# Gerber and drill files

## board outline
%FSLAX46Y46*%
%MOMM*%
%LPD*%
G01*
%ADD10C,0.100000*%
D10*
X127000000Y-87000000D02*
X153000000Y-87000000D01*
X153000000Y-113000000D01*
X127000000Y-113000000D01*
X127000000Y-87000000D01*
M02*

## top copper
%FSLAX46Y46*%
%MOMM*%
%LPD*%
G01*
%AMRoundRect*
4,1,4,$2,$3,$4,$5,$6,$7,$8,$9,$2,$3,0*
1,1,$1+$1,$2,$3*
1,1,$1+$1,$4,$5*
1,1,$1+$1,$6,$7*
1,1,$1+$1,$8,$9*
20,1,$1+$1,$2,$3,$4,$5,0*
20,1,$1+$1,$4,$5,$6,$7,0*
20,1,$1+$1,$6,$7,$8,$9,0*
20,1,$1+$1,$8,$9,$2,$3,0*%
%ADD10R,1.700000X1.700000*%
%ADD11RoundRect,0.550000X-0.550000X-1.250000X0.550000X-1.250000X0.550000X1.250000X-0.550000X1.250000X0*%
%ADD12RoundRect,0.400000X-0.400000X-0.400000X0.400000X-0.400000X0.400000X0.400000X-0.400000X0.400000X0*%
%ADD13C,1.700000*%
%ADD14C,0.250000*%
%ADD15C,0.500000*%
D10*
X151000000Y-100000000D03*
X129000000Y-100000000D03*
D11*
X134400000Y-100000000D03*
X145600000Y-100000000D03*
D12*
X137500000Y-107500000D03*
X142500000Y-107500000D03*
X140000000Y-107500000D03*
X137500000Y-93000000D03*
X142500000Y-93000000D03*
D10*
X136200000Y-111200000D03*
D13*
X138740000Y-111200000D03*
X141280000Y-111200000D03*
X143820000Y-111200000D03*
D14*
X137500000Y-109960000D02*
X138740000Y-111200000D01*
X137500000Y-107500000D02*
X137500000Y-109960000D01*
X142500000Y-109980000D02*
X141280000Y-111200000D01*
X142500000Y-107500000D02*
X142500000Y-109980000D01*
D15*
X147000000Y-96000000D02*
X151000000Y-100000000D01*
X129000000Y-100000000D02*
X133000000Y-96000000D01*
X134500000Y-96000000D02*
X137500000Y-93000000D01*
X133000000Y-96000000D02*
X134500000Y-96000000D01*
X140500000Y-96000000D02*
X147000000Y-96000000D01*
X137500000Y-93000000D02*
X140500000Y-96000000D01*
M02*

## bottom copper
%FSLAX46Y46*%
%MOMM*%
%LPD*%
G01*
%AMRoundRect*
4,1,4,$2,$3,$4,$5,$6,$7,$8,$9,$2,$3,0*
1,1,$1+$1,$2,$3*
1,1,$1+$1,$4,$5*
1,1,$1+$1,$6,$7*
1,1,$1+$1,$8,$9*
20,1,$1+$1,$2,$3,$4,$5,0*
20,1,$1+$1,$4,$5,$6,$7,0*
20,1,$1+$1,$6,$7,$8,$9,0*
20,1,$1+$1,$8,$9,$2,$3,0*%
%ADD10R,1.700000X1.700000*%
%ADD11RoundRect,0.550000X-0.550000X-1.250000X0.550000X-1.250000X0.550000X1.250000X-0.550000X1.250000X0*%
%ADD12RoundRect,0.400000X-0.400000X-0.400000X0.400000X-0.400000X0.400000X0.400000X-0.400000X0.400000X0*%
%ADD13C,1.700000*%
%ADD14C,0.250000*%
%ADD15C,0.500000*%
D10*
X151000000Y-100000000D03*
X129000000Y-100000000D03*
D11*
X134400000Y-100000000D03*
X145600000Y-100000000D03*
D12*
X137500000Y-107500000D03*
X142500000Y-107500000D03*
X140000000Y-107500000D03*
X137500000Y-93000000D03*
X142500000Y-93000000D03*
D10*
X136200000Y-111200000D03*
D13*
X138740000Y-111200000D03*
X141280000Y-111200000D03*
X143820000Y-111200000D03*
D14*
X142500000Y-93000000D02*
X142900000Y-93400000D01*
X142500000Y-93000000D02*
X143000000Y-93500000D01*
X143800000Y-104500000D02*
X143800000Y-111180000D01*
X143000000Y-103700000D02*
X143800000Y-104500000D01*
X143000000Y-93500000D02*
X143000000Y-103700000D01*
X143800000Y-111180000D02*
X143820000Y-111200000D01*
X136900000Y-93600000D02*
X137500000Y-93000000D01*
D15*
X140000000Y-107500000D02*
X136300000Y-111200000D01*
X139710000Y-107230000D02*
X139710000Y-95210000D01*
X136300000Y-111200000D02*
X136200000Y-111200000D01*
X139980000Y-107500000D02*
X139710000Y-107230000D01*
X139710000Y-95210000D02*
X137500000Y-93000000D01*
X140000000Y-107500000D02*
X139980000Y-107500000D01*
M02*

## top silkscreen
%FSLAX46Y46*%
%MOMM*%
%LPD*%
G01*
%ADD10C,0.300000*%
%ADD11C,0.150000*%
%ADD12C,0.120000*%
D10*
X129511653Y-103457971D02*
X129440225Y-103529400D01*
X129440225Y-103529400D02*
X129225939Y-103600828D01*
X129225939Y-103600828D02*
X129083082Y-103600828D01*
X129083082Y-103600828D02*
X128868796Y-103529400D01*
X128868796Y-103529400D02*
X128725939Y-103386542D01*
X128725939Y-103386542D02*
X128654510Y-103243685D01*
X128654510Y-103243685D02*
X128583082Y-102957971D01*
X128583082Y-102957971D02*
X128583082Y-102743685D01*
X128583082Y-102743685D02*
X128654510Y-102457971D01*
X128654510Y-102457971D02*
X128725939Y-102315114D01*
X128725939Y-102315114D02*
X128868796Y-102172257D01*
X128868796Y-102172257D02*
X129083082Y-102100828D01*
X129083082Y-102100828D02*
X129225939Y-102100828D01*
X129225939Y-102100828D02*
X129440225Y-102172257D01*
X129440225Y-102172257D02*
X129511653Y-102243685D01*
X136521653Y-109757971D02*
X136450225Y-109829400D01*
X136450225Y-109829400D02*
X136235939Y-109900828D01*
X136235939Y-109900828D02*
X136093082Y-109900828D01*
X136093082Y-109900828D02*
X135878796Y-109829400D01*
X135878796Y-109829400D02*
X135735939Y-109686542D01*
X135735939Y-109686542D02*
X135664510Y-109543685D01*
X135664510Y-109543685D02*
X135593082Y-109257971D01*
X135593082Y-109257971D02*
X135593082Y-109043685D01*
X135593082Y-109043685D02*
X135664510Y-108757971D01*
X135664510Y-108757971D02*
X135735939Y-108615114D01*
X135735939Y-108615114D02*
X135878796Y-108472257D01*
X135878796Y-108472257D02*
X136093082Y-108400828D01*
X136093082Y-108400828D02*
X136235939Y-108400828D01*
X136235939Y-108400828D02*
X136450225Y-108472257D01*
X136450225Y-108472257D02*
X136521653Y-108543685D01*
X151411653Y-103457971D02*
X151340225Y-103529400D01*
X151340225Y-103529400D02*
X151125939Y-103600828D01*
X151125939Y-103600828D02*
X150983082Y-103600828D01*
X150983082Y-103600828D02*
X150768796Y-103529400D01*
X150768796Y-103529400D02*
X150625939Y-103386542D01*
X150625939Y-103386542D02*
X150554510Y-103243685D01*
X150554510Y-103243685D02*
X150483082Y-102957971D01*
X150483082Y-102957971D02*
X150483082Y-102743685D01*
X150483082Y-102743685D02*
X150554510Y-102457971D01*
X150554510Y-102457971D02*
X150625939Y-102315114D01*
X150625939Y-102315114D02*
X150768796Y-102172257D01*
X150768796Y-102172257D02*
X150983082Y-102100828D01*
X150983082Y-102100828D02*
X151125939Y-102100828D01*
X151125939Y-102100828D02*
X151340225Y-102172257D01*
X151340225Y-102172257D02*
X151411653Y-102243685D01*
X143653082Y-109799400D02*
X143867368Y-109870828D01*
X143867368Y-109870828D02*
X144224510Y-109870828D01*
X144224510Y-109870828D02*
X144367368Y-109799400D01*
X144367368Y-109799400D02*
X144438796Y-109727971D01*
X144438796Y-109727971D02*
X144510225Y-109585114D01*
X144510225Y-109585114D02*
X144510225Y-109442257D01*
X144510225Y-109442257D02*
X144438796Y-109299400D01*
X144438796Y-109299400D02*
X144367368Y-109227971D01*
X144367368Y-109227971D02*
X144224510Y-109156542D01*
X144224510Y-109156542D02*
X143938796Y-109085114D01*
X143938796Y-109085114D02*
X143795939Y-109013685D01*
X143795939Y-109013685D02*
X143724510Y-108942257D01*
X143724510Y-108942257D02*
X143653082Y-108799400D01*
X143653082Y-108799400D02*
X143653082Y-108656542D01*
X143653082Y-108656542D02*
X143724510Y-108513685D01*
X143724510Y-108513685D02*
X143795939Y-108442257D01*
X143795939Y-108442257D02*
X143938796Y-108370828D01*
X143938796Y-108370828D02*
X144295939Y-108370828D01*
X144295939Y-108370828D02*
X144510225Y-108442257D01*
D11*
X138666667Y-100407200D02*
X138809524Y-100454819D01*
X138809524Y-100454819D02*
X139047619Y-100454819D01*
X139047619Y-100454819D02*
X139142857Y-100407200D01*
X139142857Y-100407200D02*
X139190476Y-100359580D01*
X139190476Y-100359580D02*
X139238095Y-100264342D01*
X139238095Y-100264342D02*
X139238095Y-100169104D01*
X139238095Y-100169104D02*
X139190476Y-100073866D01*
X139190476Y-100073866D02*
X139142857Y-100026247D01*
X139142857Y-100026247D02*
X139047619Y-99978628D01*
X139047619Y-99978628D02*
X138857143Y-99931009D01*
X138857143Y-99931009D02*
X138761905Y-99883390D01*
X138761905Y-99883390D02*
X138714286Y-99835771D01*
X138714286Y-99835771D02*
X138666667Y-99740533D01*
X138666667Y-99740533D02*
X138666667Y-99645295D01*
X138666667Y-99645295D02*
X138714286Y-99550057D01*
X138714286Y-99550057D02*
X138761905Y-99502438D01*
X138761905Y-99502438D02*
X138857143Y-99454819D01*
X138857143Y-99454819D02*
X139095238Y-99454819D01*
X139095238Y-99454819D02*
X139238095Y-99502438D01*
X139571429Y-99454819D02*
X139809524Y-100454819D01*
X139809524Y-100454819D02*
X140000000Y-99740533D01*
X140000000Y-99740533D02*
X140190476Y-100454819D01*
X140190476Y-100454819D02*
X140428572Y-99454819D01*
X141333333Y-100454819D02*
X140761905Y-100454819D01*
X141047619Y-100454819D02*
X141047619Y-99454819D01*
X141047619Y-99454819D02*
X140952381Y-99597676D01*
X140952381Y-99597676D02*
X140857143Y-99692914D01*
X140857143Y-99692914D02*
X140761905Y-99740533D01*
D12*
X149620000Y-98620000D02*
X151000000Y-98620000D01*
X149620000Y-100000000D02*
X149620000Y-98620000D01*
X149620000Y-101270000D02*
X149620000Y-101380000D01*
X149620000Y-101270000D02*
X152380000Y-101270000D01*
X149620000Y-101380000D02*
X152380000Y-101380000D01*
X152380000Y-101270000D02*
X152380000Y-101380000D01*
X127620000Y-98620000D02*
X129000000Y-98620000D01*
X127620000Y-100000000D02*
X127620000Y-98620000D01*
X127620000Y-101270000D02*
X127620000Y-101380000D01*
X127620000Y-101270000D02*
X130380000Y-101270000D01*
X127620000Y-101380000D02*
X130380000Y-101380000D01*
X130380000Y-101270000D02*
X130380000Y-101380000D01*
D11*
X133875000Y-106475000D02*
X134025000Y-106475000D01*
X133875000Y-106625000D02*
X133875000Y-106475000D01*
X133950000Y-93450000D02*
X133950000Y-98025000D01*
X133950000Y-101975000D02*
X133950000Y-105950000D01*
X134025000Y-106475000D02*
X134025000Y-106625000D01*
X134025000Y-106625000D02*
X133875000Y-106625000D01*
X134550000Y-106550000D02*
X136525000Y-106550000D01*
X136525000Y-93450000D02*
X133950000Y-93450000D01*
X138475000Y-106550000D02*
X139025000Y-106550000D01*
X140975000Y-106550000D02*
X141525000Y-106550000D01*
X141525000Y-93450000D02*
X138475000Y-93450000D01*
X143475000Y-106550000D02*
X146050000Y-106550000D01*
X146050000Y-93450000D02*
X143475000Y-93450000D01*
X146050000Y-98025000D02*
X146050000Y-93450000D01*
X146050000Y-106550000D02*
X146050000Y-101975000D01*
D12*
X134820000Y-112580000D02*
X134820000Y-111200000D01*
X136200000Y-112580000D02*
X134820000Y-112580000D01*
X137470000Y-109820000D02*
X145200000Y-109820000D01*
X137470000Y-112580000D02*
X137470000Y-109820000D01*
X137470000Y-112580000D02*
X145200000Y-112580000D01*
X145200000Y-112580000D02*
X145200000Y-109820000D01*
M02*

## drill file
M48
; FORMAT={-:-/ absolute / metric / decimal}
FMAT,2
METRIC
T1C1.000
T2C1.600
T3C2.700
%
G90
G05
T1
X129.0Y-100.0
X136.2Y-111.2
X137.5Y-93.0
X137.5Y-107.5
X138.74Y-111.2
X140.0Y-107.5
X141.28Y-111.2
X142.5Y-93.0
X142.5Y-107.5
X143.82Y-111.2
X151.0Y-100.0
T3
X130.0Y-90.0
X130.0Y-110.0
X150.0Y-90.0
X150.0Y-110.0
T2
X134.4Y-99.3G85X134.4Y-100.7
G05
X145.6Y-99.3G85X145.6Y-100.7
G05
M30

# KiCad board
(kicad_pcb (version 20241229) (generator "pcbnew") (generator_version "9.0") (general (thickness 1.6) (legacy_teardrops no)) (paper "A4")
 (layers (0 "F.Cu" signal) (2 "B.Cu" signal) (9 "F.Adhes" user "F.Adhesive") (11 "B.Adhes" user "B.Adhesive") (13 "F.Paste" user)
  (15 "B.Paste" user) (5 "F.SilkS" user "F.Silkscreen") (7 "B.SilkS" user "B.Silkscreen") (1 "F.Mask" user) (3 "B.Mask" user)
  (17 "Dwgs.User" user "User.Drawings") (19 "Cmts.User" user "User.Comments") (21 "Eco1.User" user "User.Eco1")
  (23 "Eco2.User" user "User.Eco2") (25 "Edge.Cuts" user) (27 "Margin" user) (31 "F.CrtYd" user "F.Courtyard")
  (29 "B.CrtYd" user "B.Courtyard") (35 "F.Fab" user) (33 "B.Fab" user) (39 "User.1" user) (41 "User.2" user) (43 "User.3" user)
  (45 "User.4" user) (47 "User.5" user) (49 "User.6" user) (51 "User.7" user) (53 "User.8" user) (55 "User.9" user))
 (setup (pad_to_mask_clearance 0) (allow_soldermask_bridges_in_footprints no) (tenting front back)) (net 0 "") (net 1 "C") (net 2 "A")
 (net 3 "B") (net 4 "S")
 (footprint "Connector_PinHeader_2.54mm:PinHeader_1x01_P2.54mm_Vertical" (layer "F.Cu") (at 151 100)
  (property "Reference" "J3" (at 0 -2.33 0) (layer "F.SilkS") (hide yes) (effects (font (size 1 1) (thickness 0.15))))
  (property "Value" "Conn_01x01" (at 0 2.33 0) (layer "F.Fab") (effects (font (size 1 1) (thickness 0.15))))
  (fp_line (start -1.38 -1.38) (end 0 -1.38) (stroke (width 0.12) (type solid)) (layer "F.SilkS"))
  (fp_line (start -1.38 0) (end -1.38 -1.38) (stroke (width 0.12) (type solid)) (layer "F.SilkS"))
  (fp_line (start -1.38 1.27) (end -1.38 1.38) (stroke (width 0.12) (type solid)) (layer "F.SilkS"))
  (fp_line (start -1.38 1.27) (end 1.38 1.27) (stroke (width 0.12) (type solid)) (layer "F.SilkS"))
  (fp_line (start -1.38 1.38) (end 1.38 1.38) (stroke (width 0.12) (type solid)) (layer "F.SilkS"))
  (fp_line (start 1.38 1.27) (end 1.38 1.38) (stroke (width 0.12) (type solid)) (layer "F.SilkS"))
  (pad "1" thru_hole rect (at 0 0) (size 1.7 1.7) (drill 1) (layers "*.Cu" "*.Mask") (remove_unused_layers no) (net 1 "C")))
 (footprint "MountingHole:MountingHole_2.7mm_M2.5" (layer "F.Cu") (at 130 90)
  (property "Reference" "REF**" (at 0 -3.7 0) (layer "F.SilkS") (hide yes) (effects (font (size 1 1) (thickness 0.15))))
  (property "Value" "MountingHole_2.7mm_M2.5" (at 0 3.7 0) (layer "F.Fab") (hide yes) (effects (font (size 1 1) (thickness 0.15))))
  (pad "" np_thru_hole circle (at 0 0) (size 2.7 2.7) (drill 2.7) (layers "*.Cu" "*.Mask")))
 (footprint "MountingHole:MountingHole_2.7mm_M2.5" (layer "F.Cu") (at 150 110)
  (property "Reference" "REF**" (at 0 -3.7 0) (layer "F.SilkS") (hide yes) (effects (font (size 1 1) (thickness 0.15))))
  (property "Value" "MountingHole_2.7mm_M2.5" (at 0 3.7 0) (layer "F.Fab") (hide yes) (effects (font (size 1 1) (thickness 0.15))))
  (pad "" np_thru_hole circle (at 0 0) (size 2.7 2.7) (drill 2.7) (layers "*.Cu" "*.Mask")))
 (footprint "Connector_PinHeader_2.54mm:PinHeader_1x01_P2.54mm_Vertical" (layer "F.Cu") (at 129 100)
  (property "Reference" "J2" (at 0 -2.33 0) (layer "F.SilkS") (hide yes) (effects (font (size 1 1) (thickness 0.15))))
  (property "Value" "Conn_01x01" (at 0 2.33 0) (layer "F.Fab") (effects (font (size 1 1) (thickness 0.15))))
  (fp_line (start -1.38 -1.38) (end 0 -1.38) (stroke (width 0.12) (type solid)) (layer "F.SilkS"))
  (fp_line (start -1.38 0) (end -1.38 -1.38) (stroke (width 0.12) (type solid)) (layer "F.SilkS"))
  (fp_line (start -1.38 1.27) (end -1.38 1.38) (stroke (width 0.12) (type solid)) (layer "F.SilkS"))
  (fp_line (start -1.38 1.27) (end 1.38 1.27) (stroke (width 0.12) (type solid)) (layer "F.SilkS"))
  (fp_line (start -1.38 1.38) (end 1.38 1.38) (stroke (width 0.12) (type solid)) (layer "F.SilkS"))
  (fp_line (start 1.38 1.27) (end 1.38 1.38) (stroke (width 0.12) (type solid)) (layer "F.SilkS"))
  (pad "1" thru_hole rect (at 0 0) (size 1.7 1.7) (drill 1) (layers "*.Cu" "*.Mask") (remove_unused_layers no) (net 1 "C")))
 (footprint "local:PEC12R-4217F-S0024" (layer "F.Cu") (at 140 100)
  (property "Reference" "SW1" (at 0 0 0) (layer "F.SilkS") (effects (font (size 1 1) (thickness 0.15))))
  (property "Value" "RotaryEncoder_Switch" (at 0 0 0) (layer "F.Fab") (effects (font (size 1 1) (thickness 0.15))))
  (fp_line (start -6.125 6.475) (end -5.975 6.475) (stroke (width 0.15) (type solid)) (layer "F.SilkS"))
  (fp_line (start -6.125 6.625) (end -6.125 6.475) (stroke (width 0.15) (type solid)) (layer "F.SilkS"))
  (fp_line (start -6.05 -6.55) (end -6.05 -1.975) (stroke (width 0.15) (type solid)) (layer "F.SilkS"))
  (fp_line (start -6.05 1.975) (end -6.05 5.95) (stroke (width 0.15) (type solid)) (layer "F.SilkS"))
  (fp_line (start -5.975 6.475) (end -5.975 6.625) (stroke (width 0.15) (type solid)) (layer "F.SilkS"))
  (fp_line (start -5.975 6.625) (end -6.125 6.625) (stroke (width 0.15) (type solid)) (layer "F.SilkS"))
  (fp_line (start -5.45 6.55) (end -3.475 6.55) (stroke (width 0.15) (type solid)) (layer "F.SilkS"))
  (fp_line (start -3.475 -6.55) (end -6.05 -6.55) (stroke (width 0.15) (type solid)) (layer "F.SilkS"))
  (fp_line (start -1.525 6.55) (end -0.975 6.55) (stroke (width 0.15) (type solid)) (layer "F.SilkS"))
  (fp_line (start 0.975 6.55) (end 1.525 6.55) (stroke (width 0.15) (type solid)) (layer "F.SilkS"))
  (fp_line (start 1.525 -6.55) (end -1.525 -6.55) (stroke (width 0.15) (type solid)) (layer "F.SilkS"))
  (fp_line (start 3.475 6.55) (end 6.05 6.55) (stroke (width 0.15) (type solid)) (layer "F.SilkS"))
  (fp_line (start 6.05 -6.55) (end 3.475 -6.55) (stroke (width 0.15) (type solid)) (layer "F.SilkS"))
  (fp_line (start 6.05 -1.975) (end 6.05 -6.55) (stroke (width 0.15) (type solid)) (layer "F.SilkS"))
  (fp_line (start 6.05 6.55) (end 6.05 1.975) (stroke (width 0.15) (type solid)) (layer "F.SilkS"))
  (pad "1" thru_hole roundrect (at -5.6 0) (size 2.2 3.6) (drill oval 1.6 3) (layers "*.Cu" "*.Mask") (remove_unused_layers yes)
   (keep_end_layers yes) (zone_layer_connections) (roundrect_rratio 0.25))
  (pad "2" thru_hole roundrect (at 5.6 0) (size 2.2 3.6) (drill oval 1.6 3) (layers "*.Cu" "*.Mask") (remove_unused_layers yes)
   (keep_end_layers yes) (zone_layer_connections) (roundrect_rratio 0.25))
  (pad "A" thru_hole roundrect (at -2.5 7.5) (size 1.6 1.6) (drill 1) (layers "*.Cu" "*.Mask") (remove_unused_layers yes)
   (keep_end_layers yes) (zone_layer_connections) (roundrect_rratio 0.25) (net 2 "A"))
  (pad "B" thru_hole roundrect (at 2.5 7.5) (size 1.6 1.6) (drill 1) (layers "*.Cu" "*.Mask") (remove_unused_layers yes)
   (keep_end_layers yes) (zone_layer_connections) (roundrect_rratio 0.25) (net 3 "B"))
  (pad "C" thru_hole roundrect (at 0 7.5) (size 1.6 1.6) (drill 1) (layers "*.Cu" "*.Mask") (remove_unused_layers yes) (keep_end_layers yes)
   (zone_layer_connections) (roundrect_rratio 0.25) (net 1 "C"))
  (pad "S1" thru_hole roundrect (at -2.5 -7) (size 1.6 1.6) (drill 1) (layers "*.Cu" "*.Mask") (remove_unused_layers yes)
   (keep_end_layers yes) (zone_layer_connections) (roundrect_rratio 0.25) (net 1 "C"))
  (pad "S2" thru_hole roundrect (at 2.5 -7) (size 1.6 1.6) (drill 1) (layers "*.Cu" "*.Mask") (remove_unused_layers yes)
   (keep_end_layers yes) (zone_layer_connections) (roundrect_rratio 0.25) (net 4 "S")))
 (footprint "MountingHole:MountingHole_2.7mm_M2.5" (layer "F.Cu") (at 150 90)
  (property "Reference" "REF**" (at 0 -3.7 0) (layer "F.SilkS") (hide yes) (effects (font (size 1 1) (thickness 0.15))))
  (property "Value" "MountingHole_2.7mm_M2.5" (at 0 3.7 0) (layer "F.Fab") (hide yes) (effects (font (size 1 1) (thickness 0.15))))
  (pad "" np_thru_hole circle (at 0 0) (size 2.7 2.7) (drill 2.7) (layers "*.Cu" "*.Mask")))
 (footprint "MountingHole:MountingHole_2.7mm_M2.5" (layer "F.Cu") (at 130 110)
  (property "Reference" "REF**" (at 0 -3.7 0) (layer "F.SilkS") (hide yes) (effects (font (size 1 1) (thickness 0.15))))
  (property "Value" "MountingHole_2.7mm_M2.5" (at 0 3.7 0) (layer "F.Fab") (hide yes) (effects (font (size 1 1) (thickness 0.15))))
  (pad "" np_thru_hole circle (at 0 0) (size 2.7 2.7) (drill 2.7) (layers "*.Cu" "*.Mask")))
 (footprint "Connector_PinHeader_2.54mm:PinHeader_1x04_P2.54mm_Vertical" (layer "F.Cu") (at 136.2 111.2 90)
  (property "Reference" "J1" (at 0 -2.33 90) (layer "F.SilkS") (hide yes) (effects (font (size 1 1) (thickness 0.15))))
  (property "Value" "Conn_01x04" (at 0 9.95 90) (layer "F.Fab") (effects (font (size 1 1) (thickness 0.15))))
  (fp_line (start -1.38 -1.38) (end 0 -1.38) (stroke (width 0.12) (type solid)) (layer "F.SilkS"))
  (fp_line (start -1.38 0) (end -1.38 -1.38) (stroke (width 0.12) (type solid)) (layer "F.SilkS"))
  (fp_line (start 1.38 1.27) (end 1.38 9) (stroke (width 0.12) (type solid)) (layer "F.SilkS"))
  (fp_line (start -1.38 1.27) (end 1.38 1.27) (stroke (width 0.12) (type solid)) (layer "F.SilkS"))
  (fp_line (start -1.38 1.27) (end -1.38 9) (stroke (width 0.12) (type solid)) (layer "F.SilkS"))
  (fp_line (start -1.38 9) (end 1.38 9) (stroke (width 0.12) (type solid)) (layer "F.SilkS"))
  (pad "1" thru_hole rect (at 0 0 90) (size 1.7 1.7) (drill 1) (layers "*.Cu" "*.Mask") (remove_unused_layers no) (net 1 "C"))
  (pad "2" thru_hole circle (at 0 2.54 90) (size 1.7 1.7) (drill 1) (layers "*.Cu" "*.Mask") (remove_unused_layers no) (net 2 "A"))
  (pad "3" thru_hole circle (at 0 5.08 90) (size 1.7 1.7) (drill 1) (layers "*.Cu" "*.Mask") (remove_unused_layers no) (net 3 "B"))
  (pad "4" thru_hole circle (at 0 7.62 90) (size 1.7 1.7) (drill 1) (layers "*.Cu" "*.Mask") (remove_unused_layers no) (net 4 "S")))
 (gr_rect (start 127 87) (end 153 113) (stroke (width 0.1) (type default)) (fill no) (layer "Edge.Cuts"))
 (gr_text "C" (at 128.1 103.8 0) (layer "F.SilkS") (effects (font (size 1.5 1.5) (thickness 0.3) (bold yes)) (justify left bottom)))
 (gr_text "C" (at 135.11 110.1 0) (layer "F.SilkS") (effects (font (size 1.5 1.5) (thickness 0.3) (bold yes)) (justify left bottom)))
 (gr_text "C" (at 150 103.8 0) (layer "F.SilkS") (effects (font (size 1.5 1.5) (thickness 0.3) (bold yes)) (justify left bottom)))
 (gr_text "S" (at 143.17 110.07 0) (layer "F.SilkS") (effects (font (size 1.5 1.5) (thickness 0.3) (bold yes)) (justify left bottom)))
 (segment (start 137.5 109.96) (end 138.74 111.2) (width 0.25) (layer "F.Cu") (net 2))
 (segment (start 137.5 107.5) (end 137.5 109.96) (width 0.25) (layer "F.Cu") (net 2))
 (segment (start 142.5 109.98) (end 141.28 111.2) (width 0.25) (layer "F.Cu") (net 3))
 (segment (start 142.5 107.5) (end 142.5 109.98) (width 0.25) (layer "F.Cu") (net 3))
 (segment (start 142.5 93) (end 142.9 93.4) (width 0.25) (layer "B.Cu") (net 4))
 (segment (start 142.5 93) (end 143 93.5) (width 0.25) (layer "B.Cu") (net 4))
 (segment (start 143.8 104.5) (end 143.8 111.18) (width 0.25) (layer "B.Cu") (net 4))
 (segment (start 143 103.7) (end 143.8 104.5) (width 0.25) (layer "B.Cu") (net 4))
 (segment (start 143 93.5) (end 143 103.7) (width 0.25) (layer "B.Cu") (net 4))
 (segment (start 143.8 111.18) (end 143.82 111.2) (width 0.25) (layer "B.Cu") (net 4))
 (segment (start 147 96) (end 151 100) (width 0.5) (layer "F.Cu") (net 1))
 (segment (start 129 100) (end 133 96) (width 0.5) (layer "F.Cu") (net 1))
 (segment (start 134.5 96) (end 137.5 93) (width 0.5) (layer "F.Cu") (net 1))
 (segment (start 133 96) (end 134.5 96) (width 0.5) (layer "F.Cu") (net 1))
 (segment (start 140.5 96) (end 147 96) (width 0.5) (layer "F.Cu") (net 1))
 (segment (start 137.5 93) (end 140.5 96) (width 0.5) (layer "F.Cu") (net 1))
 (segment (start 136.9 93.6) (end 137.5 93) (width 0.25) (layer "B.Cu") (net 1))
 (segment (start 140 107.5) (end 136.3 111.2) (width 0.5) (layer "B.Cu") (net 1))
 (segment (start 139.71 107.23) (end 139.71 95.21) (width 0.5) (layer "B.Cu") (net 1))
 (segment (start 136.3 111.2) (end 136.2 111.2) (width 0.5) (layer "B.Cu") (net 1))
 (segment (start 139.98 107.5) (end 139.71 107.23) (width 0.5) (layer "B.Cu") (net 1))
 (segment (start 139.71 95.21) (end 137.5 93) (width 0.5) (layer "B.Cu") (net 1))
 (segment (start 140 107.5) (end 139.98 107.5) (width 0.5) (layer "B.Cu") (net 1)))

